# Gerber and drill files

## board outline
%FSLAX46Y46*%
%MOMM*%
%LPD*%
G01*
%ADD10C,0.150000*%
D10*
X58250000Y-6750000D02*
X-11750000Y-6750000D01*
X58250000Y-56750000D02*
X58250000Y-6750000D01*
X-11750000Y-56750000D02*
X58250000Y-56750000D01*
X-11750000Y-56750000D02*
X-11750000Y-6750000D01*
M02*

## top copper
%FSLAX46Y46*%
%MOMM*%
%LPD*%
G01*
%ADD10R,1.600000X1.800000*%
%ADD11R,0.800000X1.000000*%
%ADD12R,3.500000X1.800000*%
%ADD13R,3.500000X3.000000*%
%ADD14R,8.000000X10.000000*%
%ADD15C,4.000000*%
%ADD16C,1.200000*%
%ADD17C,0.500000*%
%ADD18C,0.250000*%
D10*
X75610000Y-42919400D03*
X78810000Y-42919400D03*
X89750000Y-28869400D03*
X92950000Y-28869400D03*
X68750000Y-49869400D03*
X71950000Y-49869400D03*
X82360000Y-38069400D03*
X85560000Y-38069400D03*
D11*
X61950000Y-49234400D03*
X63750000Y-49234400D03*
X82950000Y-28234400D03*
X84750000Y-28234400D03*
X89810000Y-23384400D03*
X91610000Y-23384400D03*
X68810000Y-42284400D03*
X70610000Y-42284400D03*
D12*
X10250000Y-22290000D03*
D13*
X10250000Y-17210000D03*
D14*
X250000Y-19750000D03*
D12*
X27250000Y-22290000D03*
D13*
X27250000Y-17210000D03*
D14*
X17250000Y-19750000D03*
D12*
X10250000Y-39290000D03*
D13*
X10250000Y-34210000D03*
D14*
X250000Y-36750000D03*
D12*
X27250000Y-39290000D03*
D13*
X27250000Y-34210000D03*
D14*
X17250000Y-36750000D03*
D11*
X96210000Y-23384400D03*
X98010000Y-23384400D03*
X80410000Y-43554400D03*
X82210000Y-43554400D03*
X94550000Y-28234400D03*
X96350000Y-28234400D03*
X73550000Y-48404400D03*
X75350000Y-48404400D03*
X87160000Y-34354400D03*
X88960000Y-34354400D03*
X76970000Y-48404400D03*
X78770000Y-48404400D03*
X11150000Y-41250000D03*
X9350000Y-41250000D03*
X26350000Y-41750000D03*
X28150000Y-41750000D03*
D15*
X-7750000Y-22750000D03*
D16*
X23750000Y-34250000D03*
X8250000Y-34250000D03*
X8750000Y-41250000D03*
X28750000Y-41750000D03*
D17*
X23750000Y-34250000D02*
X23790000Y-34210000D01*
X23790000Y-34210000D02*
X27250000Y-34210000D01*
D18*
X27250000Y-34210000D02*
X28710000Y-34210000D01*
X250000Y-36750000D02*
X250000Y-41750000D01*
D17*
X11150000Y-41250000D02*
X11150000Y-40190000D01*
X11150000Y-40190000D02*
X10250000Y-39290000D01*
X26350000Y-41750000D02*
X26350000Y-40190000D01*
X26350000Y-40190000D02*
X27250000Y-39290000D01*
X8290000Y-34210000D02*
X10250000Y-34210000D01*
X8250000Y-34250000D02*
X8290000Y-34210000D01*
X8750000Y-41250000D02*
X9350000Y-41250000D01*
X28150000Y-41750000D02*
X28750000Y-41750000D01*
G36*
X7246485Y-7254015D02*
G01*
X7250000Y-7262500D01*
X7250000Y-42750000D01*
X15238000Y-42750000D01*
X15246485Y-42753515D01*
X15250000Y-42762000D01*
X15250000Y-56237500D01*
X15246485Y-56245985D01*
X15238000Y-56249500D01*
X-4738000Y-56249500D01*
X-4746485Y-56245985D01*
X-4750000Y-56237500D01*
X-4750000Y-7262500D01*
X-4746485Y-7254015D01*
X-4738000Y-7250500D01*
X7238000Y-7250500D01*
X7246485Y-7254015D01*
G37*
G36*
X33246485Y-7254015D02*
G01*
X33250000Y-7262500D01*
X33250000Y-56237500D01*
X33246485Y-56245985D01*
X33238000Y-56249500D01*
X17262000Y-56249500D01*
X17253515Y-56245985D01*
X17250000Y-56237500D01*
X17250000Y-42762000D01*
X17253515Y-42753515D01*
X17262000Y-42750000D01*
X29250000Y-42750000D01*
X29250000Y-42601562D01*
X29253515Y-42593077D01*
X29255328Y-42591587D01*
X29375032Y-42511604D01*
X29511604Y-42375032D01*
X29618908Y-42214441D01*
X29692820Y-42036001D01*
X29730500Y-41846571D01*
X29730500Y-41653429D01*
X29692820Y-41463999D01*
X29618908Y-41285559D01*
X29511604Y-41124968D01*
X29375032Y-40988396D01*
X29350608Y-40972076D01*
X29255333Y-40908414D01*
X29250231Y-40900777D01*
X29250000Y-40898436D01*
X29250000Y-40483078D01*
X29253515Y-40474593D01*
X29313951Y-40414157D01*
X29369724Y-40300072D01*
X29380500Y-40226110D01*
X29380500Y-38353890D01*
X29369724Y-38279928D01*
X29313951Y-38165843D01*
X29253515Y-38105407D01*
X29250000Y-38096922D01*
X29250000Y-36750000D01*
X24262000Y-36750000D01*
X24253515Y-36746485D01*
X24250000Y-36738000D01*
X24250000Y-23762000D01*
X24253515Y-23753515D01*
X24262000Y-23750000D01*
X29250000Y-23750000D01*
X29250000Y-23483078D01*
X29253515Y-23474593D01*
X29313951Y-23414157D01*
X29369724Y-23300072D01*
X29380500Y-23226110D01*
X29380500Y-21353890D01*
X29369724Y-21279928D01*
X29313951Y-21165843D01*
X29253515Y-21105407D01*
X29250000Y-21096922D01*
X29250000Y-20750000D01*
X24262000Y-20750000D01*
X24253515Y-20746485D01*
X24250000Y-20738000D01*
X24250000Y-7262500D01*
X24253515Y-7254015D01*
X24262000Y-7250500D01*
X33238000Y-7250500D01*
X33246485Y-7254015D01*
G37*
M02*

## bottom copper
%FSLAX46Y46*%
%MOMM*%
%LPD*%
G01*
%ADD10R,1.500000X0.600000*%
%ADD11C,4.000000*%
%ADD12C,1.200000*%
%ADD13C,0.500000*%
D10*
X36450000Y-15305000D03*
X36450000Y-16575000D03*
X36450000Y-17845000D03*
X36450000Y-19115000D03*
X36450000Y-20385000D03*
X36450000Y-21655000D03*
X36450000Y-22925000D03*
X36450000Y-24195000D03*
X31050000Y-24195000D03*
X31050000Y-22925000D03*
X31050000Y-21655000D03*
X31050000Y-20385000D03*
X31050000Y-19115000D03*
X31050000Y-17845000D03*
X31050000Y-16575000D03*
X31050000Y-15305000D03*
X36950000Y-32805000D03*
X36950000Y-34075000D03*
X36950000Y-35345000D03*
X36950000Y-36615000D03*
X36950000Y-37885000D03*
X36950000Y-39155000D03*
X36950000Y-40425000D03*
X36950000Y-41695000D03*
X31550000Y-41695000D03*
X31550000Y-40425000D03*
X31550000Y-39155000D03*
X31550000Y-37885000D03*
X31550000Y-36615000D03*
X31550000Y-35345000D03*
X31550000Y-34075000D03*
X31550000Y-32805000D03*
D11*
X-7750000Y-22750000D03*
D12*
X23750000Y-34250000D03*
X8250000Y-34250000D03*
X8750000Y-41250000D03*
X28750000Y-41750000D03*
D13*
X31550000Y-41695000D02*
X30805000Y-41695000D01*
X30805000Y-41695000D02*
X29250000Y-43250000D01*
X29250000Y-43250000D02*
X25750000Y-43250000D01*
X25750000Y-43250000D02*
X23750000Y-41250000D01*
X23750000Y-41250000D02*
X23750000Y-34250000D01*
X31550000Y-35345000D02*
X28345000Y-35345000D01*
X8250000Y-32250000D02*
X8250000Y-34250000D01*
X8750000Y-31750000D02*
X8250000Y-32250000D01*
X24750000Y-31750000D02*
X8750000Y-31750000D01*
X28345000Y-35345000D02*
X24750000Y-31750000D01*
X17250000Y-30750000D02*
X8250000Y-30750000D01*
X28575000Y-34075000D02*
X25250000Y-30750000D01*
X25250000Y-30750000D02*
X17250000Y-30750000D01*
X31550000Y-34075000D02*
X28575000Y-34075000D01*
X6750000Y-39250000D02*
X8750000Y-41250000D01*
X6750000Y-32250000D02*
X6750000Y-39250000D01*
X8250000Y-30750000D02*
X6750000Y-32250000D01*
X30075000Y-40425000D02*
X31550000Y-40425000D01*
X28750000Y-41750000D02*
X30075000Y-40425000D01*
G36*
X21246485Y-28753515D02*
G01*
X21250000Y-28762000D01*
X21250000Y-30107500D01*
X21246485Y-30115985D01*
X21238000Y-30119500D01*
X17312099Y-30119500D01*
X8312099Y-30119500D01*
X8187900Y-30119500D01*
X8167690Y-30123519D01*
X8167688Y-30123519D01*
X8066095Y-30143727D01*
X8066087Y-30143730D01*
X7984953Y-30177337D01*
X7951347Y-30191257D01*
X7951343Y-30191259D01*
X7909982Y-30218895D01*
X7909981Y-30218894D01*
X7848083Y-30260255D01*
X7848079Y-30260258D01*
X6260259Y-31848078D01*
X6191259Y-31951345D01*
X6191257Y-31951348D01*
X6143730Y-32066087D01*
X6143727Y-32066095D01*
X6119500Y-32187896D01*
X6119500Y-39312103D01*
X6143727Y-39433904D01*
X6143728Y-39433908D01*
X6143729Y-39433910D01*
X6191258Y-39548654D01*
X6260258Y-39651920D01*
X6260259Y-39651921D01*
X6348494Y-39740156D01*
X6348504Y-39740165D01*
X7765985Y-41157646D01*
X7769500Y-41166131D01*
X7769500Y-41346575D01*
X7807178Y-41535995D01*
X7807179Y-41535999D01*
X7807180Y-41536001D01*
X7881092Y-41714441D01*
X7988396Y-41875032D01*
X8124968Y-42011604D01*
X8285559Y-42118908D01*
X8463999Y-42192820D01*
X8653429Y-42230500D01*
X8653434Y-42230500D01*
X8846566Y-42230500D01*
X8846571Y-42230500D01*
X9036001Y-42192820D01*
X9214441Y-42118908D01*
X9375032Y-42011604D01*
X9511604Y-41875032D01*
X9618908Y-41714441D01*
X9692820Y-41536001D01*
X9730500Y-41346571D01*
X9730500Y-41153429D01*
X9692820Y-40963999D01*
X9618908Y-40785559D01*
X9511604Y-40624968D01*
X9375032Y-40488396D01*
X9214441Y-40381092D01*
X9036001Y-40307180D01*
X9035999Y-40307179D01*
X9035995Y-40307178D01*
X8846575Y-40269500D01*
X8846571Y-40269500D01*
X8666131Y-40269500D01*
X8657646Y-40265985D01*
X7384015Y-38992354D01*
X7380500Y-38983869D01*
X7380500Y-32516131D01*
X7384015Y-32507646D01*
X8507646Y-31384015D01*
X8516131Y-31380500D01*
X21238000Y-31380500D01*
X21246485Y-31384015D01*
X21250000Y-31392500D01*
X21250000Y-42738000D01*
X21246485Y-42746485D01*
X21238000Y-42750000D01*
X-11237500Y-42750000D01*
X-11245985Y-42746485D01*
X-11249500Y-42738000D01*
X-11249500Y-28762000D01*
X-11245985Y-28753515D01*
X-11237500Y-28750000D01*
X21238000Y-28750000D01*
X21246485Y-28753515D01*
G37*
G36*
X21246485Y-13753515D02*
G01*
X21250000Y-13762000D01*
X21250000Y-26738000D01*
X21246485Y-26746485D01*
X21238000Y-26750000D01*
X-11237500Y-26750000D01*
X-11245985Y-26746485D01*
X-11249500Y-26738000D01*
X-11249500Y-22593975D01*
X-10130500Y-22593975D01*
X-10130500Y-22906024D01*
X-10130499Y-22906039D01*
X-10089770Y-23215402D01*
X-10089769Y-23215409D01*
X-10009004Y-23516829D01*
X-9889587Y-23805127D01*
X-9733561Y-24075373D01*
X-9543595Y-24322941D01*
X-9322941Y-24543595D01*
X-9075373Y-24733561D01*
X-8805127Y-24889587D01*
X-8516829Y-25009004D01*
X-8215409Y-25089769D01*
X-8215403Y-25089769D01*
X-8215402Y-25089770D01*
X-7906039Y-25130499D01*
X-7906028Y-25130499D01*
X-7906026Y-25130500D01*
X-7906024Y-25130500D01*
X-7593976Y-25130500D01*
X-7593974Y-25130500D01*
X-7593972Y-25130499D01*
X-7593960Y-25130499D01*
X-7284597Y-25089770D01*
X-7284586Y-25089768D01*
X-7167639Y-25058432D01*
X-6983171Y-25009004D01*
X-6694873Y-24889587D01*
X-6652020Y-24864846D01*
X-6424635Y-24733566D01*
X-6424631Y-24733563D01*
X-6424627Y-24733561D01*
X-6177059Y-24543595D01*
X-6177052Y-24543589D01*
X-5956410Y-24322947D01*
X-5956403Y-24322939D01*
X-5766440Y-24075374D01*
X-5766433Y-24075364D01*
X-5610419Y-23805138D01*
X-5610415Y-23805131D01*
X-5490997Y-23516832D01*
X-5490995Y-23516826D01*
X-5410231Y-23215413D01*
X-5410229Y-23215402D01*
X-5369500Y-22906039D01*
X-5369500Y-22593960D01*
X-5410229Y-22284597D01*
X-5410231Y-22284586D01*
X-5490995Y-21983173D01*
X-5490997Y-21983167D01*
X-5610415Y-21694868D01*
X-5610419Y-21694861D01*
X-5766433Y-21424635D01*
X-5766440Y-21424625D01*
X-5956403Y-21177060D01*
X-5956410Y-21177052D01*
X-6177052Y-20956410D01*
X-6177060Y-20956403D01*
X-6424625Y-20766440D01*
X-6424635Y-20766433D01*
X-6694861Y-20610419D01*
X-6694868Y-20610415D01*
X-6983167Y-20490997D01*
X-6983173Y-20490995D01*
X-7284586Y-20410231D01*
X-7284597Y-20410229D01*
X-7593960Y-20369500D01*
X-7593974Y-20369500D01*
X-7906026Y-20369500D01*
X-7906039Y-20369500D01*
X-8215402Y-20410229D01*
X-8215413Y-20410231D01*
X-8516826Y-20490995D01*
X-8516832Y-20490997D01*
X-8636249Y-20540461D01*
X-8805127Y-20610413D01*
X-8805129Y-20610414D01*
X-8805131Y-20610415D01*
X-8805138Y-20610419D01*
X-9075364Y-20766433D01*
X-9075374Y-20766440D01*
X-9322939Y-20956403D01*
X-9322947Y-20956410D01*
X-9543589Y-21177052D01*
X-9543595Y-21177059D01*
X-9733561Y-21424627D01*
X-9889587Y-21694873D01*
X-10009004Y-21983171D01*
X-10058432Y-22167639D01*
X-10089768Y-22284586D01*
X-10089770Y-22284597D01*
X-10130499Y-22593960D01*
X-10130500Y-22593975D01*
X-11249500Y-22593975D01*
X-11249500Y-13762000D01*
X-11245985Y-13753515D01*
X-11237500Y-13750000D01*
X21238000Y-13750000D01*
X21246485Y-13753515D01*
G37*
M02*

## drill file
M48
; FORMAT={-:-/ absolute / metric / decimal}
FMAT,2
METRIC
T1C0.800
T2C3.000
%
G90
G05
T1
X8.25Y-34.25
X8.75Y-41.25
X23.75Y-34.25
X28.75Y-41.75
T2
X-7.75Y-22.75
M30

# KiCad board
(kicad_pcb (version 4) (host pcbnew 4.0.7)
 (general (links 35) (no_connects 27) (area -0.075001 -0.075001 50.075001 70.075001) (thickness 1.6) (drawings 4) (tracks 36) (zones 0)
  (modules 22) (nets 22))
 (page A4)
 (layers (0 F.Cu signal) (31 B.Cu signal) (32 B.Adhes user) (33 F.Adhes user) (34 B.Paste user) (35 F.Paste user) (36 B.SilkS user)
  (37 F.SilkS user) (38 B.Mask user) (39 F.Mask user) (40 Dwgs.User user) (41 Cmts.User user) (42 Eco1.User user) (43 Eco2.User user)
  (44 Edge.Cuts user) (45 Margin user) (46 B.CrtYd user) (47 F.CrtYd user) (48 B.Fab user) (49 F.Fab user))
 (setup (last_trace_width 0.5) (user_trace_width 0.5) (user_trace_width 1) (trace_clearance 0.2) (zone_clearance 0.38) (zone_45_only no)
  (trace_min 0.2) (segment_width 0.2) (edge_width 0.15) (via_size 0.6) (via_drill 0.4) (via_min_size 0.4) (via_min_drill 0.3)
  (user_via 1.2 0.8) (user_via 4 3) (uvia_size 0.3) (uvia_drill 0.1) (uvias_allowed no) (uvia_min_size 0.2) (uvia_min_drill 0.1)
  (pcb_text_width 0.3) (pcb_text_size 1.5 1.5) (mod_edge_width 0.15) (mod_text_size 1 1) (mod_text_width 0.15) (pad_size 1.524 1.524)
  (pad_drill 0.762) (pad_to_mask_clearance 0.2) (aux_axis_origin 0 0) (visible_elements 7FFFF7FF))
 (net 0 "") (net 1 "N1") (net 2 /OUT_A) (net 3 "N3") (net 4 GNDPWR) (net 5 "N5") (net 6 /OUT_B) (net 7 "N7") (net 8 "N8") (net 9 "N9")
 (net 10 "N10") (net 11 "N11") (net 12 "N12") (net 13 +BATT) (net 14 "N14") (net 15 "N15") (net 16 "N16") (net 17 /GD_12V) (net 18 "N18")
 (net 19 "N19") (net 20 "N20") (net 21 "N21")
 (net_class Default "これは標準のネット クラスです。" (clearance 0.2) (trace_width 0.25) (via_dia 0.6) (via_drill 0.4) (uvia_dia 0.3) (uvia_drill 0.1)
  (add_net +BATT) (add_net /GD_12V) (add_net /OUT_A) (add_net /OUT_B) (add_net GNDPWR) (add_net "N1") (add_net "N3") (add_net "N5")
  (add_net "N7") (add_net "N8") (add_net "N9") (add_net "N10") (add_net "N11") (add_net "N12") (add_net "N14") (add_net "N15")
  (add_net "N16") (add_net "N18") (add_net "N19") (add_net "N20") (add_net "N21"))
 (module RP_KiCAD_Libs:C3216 (layer F.Cu) (at 77.21 42.9194)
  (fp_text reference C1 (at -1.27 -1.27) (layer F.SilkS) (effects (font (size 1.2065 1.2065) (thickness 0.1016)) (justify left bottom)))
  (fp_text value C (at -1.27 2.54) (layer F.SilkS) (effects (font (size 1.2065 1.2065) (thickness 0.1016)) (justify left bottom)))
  (pad 1 smd rect (at -1.6 0) (size 1.6 1.8) (layers F.Cu F.Paste F.Mask) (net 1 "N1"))
  (pad 2 smd rect (at 1.6 0) (size 1.6 1.8) (layers F.Cu F.Paste F.Mask) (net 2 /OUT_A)))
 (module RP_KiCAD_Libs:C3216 (layer F.Cu) (at 91.35 28.8694)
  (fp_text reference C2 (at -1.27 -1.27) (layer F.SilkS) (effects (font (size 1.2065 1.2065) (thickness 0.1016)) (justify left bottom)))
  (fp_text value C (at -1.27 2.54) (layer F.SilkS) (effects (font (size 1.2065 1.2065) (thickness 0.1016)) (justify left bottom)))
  (pad 1 smd rect (at -1.6 0) (size 1.6 1.8) (layers F.Cu F.Paste F.Mask) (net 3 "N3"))
  (pad 2 smd rect (at 1.6 0) (size 1.6 1.8) (layers F.Cu F.Paste F.Mask) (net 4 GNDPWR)))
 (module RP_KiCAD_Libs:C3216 (layer F.Cu) (at 70.35 49.8694)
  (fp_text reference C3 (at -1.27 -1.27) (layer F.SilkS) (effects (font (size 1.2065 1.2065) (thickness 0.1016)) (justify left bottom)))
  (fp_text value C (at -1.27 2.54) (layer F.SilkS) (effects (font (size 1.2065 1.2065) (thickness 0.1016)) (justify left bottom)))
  (pad 1 smd rect (at -1.6 0) (size 1.6 1.8) (layers F.Cu F.Paste F.Mask) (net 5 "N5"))
  (pad 2 smd rect (at 1.6 0) (size 1.6 1.8) (layers F.Cu F.Paste F.Mask) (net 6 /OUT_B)))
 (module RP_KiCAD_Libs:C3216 (layer F.Cu) (at 83.96 38.0694)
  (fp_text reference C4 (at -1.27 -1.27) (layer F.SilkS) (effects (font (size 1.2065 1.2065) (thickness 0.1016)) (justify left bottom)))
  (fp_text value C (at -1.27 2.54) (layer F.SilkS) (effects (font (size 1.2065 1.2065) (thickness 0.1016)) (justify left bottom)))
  (pad 1 smd rect (at -1.6 0) (size 1.6 1.8) (layers F.Cu F.Paste F.Mask) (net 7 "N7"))
  (pad 2 smd rect (at 1.6 0) (size 1.6 1.8) (layers F.Cu F.Paste F.Mask) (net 4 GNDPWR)))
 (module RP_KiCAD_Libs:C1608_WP (layer F.Cu) (at 62.85 49.2344)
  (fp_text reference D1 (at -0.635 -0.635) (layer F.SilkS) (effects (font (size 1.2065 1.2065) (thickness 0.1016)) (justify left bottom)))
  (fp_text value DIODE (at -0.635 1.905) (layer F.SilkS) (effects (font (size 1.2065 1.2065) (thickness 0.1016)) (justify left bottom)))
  (pad 1 smd rect (at -0.9 0) (size 0.8 1) (layers F.Cu F.Paste F.Mask) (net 1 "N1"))
  (pad 2 smd rect (at 0.9 0) (size 0.8 1) (layers F.Cu F.Paste F.Mask) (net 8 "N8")))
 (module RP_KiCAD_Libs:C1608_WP (layer F.Cu) (at 83.85 28.2344)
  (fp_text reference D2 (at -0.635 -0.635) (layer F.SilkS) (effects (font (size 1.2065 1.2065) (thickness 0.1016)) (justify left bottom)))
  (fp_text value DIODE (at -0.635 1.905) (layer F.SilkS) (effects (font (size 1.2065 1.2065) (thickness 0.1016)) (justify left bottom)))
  (pad 1 smd rect (at -0.9 0) (size 0.8 1) (layers F.Cu F.Paste F.Mask) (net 3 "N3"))
  (pad 2 smd rect (at 0.9 0) (size 0.8 1) (layers F.Cu F.Paste F.Mask) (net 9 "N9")))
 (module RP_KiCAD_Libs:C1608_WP (layer F.Cu) (at 90.71 23.3844)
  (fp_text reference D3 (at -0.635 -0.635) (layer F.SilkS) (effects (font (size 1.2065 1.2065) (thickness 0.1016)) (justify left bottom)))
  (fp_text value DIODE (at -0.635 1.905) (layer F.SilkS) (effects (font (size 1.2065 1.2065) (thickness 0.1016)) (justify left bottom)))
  (pad 1 smd rect (at -0.9 0) (size 0.8 1) (layers F.Cu F.Paste F.Mask) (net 5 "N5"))
  (pad 2 smd rect (at 0.9 0) (size 0.8 1) (layers F.Cu F.Paste F.Mask) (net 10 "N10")))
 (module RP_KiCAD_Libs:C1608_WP (layer F.Cu) (at 69.71 42.2844)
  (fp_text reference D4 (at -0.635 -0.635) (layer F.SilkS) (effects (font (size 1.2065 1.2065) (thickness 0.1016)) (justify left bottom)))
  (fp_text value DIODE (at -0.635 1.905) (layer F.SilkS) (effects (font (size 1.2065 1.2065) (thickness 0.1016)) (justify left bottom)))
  (pad 1 smd rect (at -0.9 0) (size 0.8 1) (layers F.Cu F.Paste F.Mask) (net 7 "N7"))
  (pad 2 smd rect (at 0.9 0) (size 0.8 1) (layers F.Cu F.Paste F.Mask) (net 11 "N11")))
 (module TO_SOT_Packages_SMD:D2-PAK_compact (layer F.Cu) (at 7.25 19.75 90)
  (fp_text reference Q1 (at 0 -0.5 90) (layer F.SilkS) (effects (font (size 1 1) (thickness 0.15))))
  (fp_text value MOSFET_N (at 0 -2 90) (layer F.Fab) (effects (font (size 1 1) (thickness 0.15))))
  (pad G smd rect (at -2.54 3 90) (size 1.8 3.5) (layers F.Cu F.Paste F.Mask) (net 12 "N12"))
  (pad S smd rect (at 2.54 3 90) (size 3 3.5) (layers F.Cu F.Paste F.Mask) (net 2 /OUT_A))
  (pad D smd rect (at 0 -7 90) (size 10 8) (layers F.Cu F.Paste F.Mask) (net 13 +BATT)))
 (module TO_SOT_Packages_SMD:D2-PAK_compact (layer F.Cu) (at 24.25 19.75 90)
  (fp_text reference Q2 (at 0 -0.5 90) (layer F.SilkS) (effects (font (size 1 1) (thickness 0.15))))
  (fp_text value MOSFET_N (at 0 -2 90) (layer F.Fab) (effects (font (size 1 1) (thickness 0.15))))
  (pad G smd rect (at -2.54 3 90) (size 1.8 3.5) (layers F.Cu F.Paste F.Mask) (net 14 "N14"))
  (pad S smd rect (at 2.54 3 90) (size 3 3.5) (layers F.Cu F.Paste F.Mask) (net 4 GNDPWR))
  (pad D smd rect (at 0 -7 90) (size 10 8) (layers F.Cu F.Paste F.Mask) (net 2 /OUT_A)))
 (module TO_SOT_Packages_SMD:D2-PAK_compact (layer F.Cu) (at 7.25 36.75 90)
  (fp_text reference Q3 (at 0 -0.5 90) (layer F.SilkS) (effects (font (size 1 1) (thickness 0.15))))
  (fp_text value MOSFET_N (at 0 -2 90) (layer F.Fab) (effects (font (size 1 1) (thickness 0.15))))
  (pad G smd rect (at -2.54 3 90) (size 1.8 3.5) (layers F.Cu F.Paste F.Mask) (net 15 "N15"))
  (pad S smd rect (at 2.54 3 90) (size 3 3.5) (layers F.Cu F.Paste F.Mask) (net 6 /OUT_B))
  (pad D smd rect (at 0 -7 90) (size 10 8) (layers F.Cu F.Paste F.Mask) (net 13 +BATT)))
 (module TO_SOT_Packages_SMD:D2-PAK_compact (layer F.Cu) (at 24.25 36.75 90)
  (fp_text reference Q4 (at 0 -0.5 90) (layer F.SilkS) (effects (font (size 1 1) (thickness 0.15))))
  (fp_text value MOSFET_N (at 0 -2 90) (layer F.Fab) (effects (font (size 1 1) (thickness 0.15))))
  (pad G smd rect (at -2.54 3 90) (size 1.8 3.5) (layers F.Cu F.Paste F.Mask) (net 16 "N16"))
  (pad S smd rect (at 2.54 3 90) (size 3 3.5) (layers F.Cu F.Paste F.Mask) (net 4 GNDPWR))
  (pad D smd rect (at 0 -7 90) (size 10 8) (layers F.Cu F.Paste F.Mask) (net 6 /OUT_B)))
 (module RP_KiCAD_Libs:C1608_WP (layer F.Cu) (at 97.11 23.3844)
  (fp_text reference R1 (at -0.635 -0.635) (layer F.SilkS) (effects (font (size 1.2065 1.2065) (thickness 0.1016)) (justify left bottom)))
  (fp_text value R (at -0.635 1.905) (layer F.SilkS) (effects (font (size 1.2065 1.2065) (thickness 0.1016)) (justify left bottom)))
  (pad 1 smd rect (at -0.9 0) (size 0.8 1) (layers F.Cu F.Paste F.Mask) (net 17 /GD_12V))
  (pad 2 smd rect (at 0.9 0) (size 0.8 1) (layers F.Cu F.Paste F.Mask) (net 8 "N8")))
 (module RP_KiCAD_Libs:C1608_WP (layer F.Cu) (at 81.31 43.5544)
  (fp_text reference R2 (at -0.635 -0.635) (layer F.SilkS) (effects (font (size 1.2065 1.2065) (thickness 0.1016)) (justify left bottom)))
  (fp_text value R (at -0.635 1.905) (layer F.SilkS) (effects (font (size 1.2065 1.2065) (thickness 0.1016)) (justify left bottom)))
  (pad 1 smd rect (at -0.9 0) (size 0.8 1) (layers F.Cu F.Paste F.Mask) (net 17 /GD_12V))
  (pad 2 smd rect (at 0.9 0) (size 0.8 1) (layers F.Cu F.Paste F.Mask) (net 9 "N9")))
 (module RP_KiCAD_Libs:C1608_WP (layer F.Cu) (at 95.45 28.2344)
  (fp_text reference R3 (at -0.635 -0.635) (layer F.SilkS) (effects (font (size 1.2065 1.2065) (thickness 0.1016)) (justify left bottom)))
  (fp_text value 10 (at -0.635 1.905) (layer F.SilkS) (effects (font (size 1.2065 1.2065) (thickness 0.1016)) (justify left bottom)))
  (pad 1 smd rect (at -0.9 0) (size 0.8 1) (layers F.Cu F.Paste F.Mask) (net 12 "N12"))
  (pad 2 smd rect (at 0.9 0) (size 0.8 1) (layers F.Cu F.Paste F.Mask) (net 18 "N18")))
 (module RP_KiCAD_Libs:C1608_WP (layer F.Cu) (at 74.45 48.4044)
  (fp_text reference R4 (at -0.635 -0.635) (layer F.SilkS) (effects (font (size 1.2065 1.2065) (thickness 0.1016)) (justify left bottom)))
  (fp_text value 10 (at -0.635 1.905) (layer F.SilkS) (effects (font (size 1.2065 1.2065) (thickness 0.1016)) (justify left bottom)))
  (pad 1 smd rect (at -0.9 0) (size 0.8 1) (layers F.Cu F.Paste F.Mask) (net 14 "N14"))
  (pad 2 smd rect (at 0.9 0) (size 0.8 1) (layers F.Cu F.Paste F.Mask) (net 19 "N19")))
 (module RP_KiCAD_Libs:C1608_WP (layer F.Cu) (at 88.06 34.3544)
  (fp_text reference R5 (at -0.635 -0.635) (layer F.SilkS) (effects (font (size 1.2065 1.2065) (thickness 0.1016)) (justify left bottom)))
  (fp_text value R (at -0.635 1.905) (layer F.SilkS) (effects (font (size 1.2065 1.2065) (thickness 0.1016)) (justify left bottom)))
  (pad 1 smd rect (at -0.9 0) (size 0.8 1) (layers F.Cu F.Paste F.Mask) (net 17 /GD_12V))
  (pad 2 smd rect (at 0.9 0) (size 0.8 1) (layers F.Cu F.Paste F.Mask) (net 10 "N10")))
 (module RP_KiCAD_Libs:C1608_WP (layer F.Cu) (at 77.87 48.4044)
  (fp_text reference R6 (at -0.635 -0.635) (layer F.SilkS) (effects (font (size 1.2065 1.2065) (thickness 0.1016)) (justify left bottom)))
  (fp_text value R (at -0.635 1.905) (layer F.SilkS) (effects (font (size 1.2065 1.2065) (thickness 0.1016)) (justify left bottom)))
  (pad 1 smd rect (at -0.9 0) (size 0.8 1) (layers F.Cu F.Paste F.Mask) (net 17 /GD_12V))
  (pad 2 smd rect (at 0.9 0) (size 0.8 1) (layers F.Cu F.Paste F.Mask) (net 11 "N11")))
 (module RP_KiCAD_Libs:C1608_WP (layer F.Cu) (at 10.25 41.25 180)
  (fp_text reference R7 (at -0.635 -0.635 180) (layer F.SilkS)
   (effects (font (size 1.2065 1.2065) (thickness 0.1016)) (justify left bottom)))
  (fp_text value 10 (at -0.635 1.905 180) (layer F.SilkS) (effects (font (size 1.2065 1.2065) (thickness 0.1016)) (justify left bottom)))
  (pad 1 smd rect (at -0.9 0 180) (size 0.8 1) (layers F.Cu F.Paste F.Mask) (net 15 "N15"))
  (pad 2 smd rect (at 0.9 0 180) (size 0.8 1) (layers F.Cu F.Paste F.Mask) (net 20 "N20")))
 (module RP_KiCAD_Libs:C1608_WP (layer F.Cu) (at 27.25 41.75)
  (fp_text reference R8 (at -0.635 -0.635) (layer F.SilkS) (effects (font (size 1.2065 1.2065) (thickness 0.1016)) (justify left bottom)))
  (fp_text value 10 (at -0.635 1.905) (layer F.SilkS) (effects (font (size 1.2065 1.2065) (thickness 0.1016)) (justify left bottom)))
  (pad 1 smd rect (at -0.9 0) (size 0.8 1) (layers F.Cu F.Paste F.Mask) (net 16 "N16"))
  (pad 2 smd rect (at 0.9 0) (size 0.8 1) (layers F.Cu F.Paste F.Mask) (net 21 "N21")))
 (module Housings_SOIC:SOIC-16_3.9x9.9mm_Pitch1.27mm (layer B.Cu) (at 33.75 19.75 180)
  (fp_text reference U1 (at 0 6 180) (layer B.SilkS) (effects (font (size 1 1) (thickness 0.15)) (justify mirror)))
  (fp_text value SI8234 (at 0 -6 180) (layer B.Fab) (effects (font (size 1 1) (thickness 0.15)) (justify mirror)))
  (pad 1 smd rect (at -2.7 4.445 180) (size 1.5 0.6) (layers B.Cu B.Paste B.Mask))
  (pad 2 smd rect (at -2.7 3.175 180) (size 1.5 0.6) (layers B.Cu B.Paste B.Mask))
  (pad 3 smd rect (at -2.7 1.905 180) (size 1.5 0.6) (layers B.Cu B.Paste B.Mask))
  (pad 4 smd rect (at -2.7 0.635 180) (size 1.5 0.6) (layers B.Cu B.Paste B.Mask))
  (pad 5 smd rect (at -2.7 -0.635 180) (size 1.5 0.6) (layers B.Cu B.Paste B.Mask))
  (pad 6 smd rect (at -2.7 -1.905 180) (size 1.5 0.6) (layers B.Cu B.Paste B.Mask))
  (pad 7 smd rect (at -2.7 -3.175 180) (size 1.5 0.6) (layers B.Cu B.Paste B.Mask))
  (pad 8 smd rect (at -2.7 -4.445 180) (size 1.5 0.6) (layers B.Cu B.Paste B.Mask))
  (pad 9 smd rect (at 2.7 -4.445 180) (size 1.5 0.6) (layers B.Cu B.Paste B.Mask) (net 4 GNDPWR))
  (pad 10 smd rect (at 2.7 -3.175 180) (size 1.5 0.6) (layers B.Cu B.Paste B.Mask) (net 19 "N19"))
  (pad 11 smd rect (at 2.7 -1.905 180) (size 1.5 0.6) (layers B.Cu B.Paste B.Mask) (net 3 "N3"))
  (pad 12 smd rect (at 2.7 -0.635 180) (size 1.5 0.6) (layers B.Cu B.Paste B.Mask))
  (pad 13 smd rect (at 2.7 0.635 180) (size 1.5 0.6) (layers B.Cu B.Paste B.Mask))
  (pad 14 smd rect (at 2.7 1.905 180) (size 1.5 0.6) (layers B.Cu B.Paste B.Mask) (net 2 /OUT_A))
  (pad 15 smd rect (at 2.7 3.175 180) (size 1.5 0.6) (layers B.Cu B.Paste B.Mask) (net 18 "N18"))
  (pad 16 smd rect (at 2.7 4.445 180) (size 1.5 0.6) (layers B.Cu B.Paste B.Mask) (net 1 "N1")))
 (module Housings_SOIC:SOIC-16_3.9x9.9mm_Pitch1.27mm (layer B.Cu) (at 34.25 37.25 180)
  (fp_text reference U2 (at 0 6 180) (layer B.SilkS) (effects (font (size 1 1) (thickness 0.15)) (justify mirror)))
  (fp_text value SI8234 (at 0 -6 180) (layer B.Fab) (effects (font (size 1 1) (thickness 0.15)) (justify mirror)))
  (pad 1 smd rect (at -2.7 4.445 180) (size 1.5 0.6) (layers B.Cu B.Paste B.Mask))
  (pad 2 smd rect (at -2.7 3.175 180) (size 1.5 0.6) (layers B.Cu B.Paste B.Mask))
  (pad 3 smd rect (at -2.7 1.905 180) (size 1.5 0.6) (layers B.Cu B.Paste B.Mask))
  (pad 4 smd rect (at -2.7 0.635 180) (size 1.5 0.6) (layers B.Cu B.Paste B.Mask))
  (pad 5 smd rect (at -2.7 -0.635 180) (size 1.5 0.6) (layers B.Cu B.Paste B.Mask))
  (pad 6 smd rect (at -2.7 -1.905 180) (size 1.5 0.6) (layers B.Cu B.Paste B.Mask))
  (pad 7 smd rect (at -2.7 -3.175 180) (size 1.5 0.6) (layers B.Cu B.Paste B.Mask))
  (pad 8 smd rect (at -2.7 -4.445 180) (size 1.5 0.6) (layers B.Cu B.Paste B.Mask))
  (pad 9 smd rect (at 2.7 -4.445 180) (size 1.5 0.6) (layers B.Cu B.Paste B.Mask) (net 4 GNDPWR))
  (pad 10 smd rect (at 2.7 -3.175 180) (size 1.5 0.6) (layers B.Cu B.Paste B.Mask) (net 21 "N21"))
  (pad 11 smd rect (at 2.7 -1.905 180) (size 1.5 0.6) (layers B.Cu B.Paste B.Mask) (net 7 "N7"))
  (pad 12 smd rect (at 2.7 -0.635 180) (size 1.5 0.6) (layers B.Cu B.Paste B.Mask))
  (pad 13 smd rect (at 2.7 0.635 180) (size 1.5 0.6) (layers B.Cu B.Paste B.Mask))
  (pad 14 smd rect (at 2.7 1.905 180) (size 1.5 0.6) (layers B.Cu B.Paste B.Mask) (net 6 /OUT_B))
  (pad 15 smd rect (at 2.7 3.175 180) (size 1.5 0.6) (layers B.Cu B.Paste B.Mask) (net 20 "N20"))
  (pad 16 smd rect (at 2.7 4.445 180) (size 1.5 0.6) (layers B.Cu B.Paste B.Mask) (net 5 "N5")))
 (gr_line (start 58.25 6.75) (end -11.75 6.75) (angle 90) (layer Edge.Cuts) (width 0.15))
 (gr_line (start 58.25 56.75) (end 58.25 6.75) (angle 90) (layer Edge.Cuts) (width 0.15))
 (gr_line (start -11.75 56.75) (end 58.25 56.75) (angle 90) (layer Edge.Cuts) (width 0.15))
 (gr_line (start -11.75 56.75) (end -11.75 6.75) (angle 90) (layer Edge.Cuts) (width 0.15))
 (via (at -7.75 22.75) (size 4) (drill 3) (layers F.Cu B.Cu) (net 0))
 (segment (start 31.55 41.695) (end 30.805 41.695) (width 0.5) (layer B.Cu) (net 4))
 (segment (start 30.805 41.695) (end 29.25 43.25) (width 0.5) (layer B.Cu) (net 4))
 (segment (start 29.25 43.25) (end 25.75 43.25) (width 0.5) (layer B.Cu) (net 4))
 (segment (start 25.75 43.25) (end 23.75 41.25) (width 0.5) (layer B.Cu) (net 4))
 (segment (start 23.75 41.25) (end 23.75 34.25) (width 0.5) (layer B.Cu) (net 4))
 (via (at 23.75 34.25) (size 1.2) (drill 0.8) (layers F.Cu B.Cu) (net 4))
 (segment (start 23.75 34.25) (end 23.79 34.21) (width 0.5) (layer F.Cu) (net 4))
 (segment (start 23.79 34.21) (end 27.25 34.21) (width 0.5) (layer F.Cu) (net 4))
 (segment (start 27.25 34.21) (end 28.71 34.21) (width 0.25) (layer F.Cu) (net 4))
 (segment (start 0.25 36.75) (end 0.25 41.75) (width 0.25) (layer F.Cu) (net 13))
 (segment (start 11.15 41.25) (end 11.15 40.19) (width 0.5) (layer F.Cu) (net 15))
 (segment (start 11.15 40.19) (end 10.25 39.29) (width 0.5) (layer F.Cu) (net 15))
 (segment (start 26.35 41.75) (end 26.35 40.19) (width 0.5) (layer F.Cu) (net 16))
 (segment (start 26.35 40.19) (end 27.25 39.29) (width 0.5) (layer F.Cu) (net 16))
 (segment (start 31.55 35.345) (end 28.345 35.345) (width 0.5) (layer B.Cu) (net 6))
 (segment (start 8.29 34.21) (end 10.25 34.21) (width 0.5) (layer F.Cu) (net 6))
 (segment (start 8.25 34.25) (end 8.29 34.21) (width 0.5) (layer F.Cu) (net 6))
 (via (at 8.25 34.25) (size 1.2) (drill 0.8) (layers F.Cu B.Cu) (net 6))
 (segment (start 8.25 32.25) (end 8.25 34.25) (width 0.5) (layer B.Cu) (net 6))
 (segment (start 8.75 31.75) (end 8.25 32.25) (width 0.5) (layer B.Cu) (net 6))
 (segment (start 24.75 31.75) (end 8.75 31.75) (width 0.5) (layer B.Cu) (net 6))
 (segment (start 28.345 35.345) (end 24.75 31.75) (width 0.5) (layer B.Cu) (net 6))
 (segment (start 17.25 30.75) (end 8.25 30.75) (width 0.5) (layer B.Cu) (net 20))
 (segment (start 28.575 34.075) (end 25.25 30.75) (width 0.5) (layer B.Cu) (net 20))
 (segment (start 25.25 30.75) (end 17.25 30.75) (width 0.5) (layer B.Cu) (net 20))
 (segment (start 31.55 34.075) (end 28.575 34.075) (width 0.5) (layer B.Cu) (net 20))
 (segment (start 8.75 41.25) (end 9.35 41.25) (width 0.5) (layer F.Cu) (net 20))
 (via (at 8.75 41.25) (size 1.2) (drill 0.8) (layers F.Cu B.Cu) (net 20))
 (segment (start 6.75 39.25) (end 8.75 41.25) (width 0.5) (layer B.Cu) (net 20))
 (segment (start 6.75 32.25) (end 6.75 39.25) (width 0.5) (layer B.Cu) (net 20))
 (segment (start 8.25 30.75) (end 6.75 32.25) (width 0.5) (layer B.Cu) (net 20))
 (segment (start 28.15 41.75) (end 28.75 41.75) (width 0.5) (layer F.Cu) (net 21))
 (segment (start 30.075 40.425) (end 31.55 40.425) (width 0.5) (layer B.Cu) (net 21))
 (segment (start 28.75 41.75) (end 30.075 40.425) (width 0.5) (layer B.Cu) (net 21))
 (via (at 28.75 41.75) (size 1.2) (drill 0.8) (layers F.Cu B.Cu) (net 21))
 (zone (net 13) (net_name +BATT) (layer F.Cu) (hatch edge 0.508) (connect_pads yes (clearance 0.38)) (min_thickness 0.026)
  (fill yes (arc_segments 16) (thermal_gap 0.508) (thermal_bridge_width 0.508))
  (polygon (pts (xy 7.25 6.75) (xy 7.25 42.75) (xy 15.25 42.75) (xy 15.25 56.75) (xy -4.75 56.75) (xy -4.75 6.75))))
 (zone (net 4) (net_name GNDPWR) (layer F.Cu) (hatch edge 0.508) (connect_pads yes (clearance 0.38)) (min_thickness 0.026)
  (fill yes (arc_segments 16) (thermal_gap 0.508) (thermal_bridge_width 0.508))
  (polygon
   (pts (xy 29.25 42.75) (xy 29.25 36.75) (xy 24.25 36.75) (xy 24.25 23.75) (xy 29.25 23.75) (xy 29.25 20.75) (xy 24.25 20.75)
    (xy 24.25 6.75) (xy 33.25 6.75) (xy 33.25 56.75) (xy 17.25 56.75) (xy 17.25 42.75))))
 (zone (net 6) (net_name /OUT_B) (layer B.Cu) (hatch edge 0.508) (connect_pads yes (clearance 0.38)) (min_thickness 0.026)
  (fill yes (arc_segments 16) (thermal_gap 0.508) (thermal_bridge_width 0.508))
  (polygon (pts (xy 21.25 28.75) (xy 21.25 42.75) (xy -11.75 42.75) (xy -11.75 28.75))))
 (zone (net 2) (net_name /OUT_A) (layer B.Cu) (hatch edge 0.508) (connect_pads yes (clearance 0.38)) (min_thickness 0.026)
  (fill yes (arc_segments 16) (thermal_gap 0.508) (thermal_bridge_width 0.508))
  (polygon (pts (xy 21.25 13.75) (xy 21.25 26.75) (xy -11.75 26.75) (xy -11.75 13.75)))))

